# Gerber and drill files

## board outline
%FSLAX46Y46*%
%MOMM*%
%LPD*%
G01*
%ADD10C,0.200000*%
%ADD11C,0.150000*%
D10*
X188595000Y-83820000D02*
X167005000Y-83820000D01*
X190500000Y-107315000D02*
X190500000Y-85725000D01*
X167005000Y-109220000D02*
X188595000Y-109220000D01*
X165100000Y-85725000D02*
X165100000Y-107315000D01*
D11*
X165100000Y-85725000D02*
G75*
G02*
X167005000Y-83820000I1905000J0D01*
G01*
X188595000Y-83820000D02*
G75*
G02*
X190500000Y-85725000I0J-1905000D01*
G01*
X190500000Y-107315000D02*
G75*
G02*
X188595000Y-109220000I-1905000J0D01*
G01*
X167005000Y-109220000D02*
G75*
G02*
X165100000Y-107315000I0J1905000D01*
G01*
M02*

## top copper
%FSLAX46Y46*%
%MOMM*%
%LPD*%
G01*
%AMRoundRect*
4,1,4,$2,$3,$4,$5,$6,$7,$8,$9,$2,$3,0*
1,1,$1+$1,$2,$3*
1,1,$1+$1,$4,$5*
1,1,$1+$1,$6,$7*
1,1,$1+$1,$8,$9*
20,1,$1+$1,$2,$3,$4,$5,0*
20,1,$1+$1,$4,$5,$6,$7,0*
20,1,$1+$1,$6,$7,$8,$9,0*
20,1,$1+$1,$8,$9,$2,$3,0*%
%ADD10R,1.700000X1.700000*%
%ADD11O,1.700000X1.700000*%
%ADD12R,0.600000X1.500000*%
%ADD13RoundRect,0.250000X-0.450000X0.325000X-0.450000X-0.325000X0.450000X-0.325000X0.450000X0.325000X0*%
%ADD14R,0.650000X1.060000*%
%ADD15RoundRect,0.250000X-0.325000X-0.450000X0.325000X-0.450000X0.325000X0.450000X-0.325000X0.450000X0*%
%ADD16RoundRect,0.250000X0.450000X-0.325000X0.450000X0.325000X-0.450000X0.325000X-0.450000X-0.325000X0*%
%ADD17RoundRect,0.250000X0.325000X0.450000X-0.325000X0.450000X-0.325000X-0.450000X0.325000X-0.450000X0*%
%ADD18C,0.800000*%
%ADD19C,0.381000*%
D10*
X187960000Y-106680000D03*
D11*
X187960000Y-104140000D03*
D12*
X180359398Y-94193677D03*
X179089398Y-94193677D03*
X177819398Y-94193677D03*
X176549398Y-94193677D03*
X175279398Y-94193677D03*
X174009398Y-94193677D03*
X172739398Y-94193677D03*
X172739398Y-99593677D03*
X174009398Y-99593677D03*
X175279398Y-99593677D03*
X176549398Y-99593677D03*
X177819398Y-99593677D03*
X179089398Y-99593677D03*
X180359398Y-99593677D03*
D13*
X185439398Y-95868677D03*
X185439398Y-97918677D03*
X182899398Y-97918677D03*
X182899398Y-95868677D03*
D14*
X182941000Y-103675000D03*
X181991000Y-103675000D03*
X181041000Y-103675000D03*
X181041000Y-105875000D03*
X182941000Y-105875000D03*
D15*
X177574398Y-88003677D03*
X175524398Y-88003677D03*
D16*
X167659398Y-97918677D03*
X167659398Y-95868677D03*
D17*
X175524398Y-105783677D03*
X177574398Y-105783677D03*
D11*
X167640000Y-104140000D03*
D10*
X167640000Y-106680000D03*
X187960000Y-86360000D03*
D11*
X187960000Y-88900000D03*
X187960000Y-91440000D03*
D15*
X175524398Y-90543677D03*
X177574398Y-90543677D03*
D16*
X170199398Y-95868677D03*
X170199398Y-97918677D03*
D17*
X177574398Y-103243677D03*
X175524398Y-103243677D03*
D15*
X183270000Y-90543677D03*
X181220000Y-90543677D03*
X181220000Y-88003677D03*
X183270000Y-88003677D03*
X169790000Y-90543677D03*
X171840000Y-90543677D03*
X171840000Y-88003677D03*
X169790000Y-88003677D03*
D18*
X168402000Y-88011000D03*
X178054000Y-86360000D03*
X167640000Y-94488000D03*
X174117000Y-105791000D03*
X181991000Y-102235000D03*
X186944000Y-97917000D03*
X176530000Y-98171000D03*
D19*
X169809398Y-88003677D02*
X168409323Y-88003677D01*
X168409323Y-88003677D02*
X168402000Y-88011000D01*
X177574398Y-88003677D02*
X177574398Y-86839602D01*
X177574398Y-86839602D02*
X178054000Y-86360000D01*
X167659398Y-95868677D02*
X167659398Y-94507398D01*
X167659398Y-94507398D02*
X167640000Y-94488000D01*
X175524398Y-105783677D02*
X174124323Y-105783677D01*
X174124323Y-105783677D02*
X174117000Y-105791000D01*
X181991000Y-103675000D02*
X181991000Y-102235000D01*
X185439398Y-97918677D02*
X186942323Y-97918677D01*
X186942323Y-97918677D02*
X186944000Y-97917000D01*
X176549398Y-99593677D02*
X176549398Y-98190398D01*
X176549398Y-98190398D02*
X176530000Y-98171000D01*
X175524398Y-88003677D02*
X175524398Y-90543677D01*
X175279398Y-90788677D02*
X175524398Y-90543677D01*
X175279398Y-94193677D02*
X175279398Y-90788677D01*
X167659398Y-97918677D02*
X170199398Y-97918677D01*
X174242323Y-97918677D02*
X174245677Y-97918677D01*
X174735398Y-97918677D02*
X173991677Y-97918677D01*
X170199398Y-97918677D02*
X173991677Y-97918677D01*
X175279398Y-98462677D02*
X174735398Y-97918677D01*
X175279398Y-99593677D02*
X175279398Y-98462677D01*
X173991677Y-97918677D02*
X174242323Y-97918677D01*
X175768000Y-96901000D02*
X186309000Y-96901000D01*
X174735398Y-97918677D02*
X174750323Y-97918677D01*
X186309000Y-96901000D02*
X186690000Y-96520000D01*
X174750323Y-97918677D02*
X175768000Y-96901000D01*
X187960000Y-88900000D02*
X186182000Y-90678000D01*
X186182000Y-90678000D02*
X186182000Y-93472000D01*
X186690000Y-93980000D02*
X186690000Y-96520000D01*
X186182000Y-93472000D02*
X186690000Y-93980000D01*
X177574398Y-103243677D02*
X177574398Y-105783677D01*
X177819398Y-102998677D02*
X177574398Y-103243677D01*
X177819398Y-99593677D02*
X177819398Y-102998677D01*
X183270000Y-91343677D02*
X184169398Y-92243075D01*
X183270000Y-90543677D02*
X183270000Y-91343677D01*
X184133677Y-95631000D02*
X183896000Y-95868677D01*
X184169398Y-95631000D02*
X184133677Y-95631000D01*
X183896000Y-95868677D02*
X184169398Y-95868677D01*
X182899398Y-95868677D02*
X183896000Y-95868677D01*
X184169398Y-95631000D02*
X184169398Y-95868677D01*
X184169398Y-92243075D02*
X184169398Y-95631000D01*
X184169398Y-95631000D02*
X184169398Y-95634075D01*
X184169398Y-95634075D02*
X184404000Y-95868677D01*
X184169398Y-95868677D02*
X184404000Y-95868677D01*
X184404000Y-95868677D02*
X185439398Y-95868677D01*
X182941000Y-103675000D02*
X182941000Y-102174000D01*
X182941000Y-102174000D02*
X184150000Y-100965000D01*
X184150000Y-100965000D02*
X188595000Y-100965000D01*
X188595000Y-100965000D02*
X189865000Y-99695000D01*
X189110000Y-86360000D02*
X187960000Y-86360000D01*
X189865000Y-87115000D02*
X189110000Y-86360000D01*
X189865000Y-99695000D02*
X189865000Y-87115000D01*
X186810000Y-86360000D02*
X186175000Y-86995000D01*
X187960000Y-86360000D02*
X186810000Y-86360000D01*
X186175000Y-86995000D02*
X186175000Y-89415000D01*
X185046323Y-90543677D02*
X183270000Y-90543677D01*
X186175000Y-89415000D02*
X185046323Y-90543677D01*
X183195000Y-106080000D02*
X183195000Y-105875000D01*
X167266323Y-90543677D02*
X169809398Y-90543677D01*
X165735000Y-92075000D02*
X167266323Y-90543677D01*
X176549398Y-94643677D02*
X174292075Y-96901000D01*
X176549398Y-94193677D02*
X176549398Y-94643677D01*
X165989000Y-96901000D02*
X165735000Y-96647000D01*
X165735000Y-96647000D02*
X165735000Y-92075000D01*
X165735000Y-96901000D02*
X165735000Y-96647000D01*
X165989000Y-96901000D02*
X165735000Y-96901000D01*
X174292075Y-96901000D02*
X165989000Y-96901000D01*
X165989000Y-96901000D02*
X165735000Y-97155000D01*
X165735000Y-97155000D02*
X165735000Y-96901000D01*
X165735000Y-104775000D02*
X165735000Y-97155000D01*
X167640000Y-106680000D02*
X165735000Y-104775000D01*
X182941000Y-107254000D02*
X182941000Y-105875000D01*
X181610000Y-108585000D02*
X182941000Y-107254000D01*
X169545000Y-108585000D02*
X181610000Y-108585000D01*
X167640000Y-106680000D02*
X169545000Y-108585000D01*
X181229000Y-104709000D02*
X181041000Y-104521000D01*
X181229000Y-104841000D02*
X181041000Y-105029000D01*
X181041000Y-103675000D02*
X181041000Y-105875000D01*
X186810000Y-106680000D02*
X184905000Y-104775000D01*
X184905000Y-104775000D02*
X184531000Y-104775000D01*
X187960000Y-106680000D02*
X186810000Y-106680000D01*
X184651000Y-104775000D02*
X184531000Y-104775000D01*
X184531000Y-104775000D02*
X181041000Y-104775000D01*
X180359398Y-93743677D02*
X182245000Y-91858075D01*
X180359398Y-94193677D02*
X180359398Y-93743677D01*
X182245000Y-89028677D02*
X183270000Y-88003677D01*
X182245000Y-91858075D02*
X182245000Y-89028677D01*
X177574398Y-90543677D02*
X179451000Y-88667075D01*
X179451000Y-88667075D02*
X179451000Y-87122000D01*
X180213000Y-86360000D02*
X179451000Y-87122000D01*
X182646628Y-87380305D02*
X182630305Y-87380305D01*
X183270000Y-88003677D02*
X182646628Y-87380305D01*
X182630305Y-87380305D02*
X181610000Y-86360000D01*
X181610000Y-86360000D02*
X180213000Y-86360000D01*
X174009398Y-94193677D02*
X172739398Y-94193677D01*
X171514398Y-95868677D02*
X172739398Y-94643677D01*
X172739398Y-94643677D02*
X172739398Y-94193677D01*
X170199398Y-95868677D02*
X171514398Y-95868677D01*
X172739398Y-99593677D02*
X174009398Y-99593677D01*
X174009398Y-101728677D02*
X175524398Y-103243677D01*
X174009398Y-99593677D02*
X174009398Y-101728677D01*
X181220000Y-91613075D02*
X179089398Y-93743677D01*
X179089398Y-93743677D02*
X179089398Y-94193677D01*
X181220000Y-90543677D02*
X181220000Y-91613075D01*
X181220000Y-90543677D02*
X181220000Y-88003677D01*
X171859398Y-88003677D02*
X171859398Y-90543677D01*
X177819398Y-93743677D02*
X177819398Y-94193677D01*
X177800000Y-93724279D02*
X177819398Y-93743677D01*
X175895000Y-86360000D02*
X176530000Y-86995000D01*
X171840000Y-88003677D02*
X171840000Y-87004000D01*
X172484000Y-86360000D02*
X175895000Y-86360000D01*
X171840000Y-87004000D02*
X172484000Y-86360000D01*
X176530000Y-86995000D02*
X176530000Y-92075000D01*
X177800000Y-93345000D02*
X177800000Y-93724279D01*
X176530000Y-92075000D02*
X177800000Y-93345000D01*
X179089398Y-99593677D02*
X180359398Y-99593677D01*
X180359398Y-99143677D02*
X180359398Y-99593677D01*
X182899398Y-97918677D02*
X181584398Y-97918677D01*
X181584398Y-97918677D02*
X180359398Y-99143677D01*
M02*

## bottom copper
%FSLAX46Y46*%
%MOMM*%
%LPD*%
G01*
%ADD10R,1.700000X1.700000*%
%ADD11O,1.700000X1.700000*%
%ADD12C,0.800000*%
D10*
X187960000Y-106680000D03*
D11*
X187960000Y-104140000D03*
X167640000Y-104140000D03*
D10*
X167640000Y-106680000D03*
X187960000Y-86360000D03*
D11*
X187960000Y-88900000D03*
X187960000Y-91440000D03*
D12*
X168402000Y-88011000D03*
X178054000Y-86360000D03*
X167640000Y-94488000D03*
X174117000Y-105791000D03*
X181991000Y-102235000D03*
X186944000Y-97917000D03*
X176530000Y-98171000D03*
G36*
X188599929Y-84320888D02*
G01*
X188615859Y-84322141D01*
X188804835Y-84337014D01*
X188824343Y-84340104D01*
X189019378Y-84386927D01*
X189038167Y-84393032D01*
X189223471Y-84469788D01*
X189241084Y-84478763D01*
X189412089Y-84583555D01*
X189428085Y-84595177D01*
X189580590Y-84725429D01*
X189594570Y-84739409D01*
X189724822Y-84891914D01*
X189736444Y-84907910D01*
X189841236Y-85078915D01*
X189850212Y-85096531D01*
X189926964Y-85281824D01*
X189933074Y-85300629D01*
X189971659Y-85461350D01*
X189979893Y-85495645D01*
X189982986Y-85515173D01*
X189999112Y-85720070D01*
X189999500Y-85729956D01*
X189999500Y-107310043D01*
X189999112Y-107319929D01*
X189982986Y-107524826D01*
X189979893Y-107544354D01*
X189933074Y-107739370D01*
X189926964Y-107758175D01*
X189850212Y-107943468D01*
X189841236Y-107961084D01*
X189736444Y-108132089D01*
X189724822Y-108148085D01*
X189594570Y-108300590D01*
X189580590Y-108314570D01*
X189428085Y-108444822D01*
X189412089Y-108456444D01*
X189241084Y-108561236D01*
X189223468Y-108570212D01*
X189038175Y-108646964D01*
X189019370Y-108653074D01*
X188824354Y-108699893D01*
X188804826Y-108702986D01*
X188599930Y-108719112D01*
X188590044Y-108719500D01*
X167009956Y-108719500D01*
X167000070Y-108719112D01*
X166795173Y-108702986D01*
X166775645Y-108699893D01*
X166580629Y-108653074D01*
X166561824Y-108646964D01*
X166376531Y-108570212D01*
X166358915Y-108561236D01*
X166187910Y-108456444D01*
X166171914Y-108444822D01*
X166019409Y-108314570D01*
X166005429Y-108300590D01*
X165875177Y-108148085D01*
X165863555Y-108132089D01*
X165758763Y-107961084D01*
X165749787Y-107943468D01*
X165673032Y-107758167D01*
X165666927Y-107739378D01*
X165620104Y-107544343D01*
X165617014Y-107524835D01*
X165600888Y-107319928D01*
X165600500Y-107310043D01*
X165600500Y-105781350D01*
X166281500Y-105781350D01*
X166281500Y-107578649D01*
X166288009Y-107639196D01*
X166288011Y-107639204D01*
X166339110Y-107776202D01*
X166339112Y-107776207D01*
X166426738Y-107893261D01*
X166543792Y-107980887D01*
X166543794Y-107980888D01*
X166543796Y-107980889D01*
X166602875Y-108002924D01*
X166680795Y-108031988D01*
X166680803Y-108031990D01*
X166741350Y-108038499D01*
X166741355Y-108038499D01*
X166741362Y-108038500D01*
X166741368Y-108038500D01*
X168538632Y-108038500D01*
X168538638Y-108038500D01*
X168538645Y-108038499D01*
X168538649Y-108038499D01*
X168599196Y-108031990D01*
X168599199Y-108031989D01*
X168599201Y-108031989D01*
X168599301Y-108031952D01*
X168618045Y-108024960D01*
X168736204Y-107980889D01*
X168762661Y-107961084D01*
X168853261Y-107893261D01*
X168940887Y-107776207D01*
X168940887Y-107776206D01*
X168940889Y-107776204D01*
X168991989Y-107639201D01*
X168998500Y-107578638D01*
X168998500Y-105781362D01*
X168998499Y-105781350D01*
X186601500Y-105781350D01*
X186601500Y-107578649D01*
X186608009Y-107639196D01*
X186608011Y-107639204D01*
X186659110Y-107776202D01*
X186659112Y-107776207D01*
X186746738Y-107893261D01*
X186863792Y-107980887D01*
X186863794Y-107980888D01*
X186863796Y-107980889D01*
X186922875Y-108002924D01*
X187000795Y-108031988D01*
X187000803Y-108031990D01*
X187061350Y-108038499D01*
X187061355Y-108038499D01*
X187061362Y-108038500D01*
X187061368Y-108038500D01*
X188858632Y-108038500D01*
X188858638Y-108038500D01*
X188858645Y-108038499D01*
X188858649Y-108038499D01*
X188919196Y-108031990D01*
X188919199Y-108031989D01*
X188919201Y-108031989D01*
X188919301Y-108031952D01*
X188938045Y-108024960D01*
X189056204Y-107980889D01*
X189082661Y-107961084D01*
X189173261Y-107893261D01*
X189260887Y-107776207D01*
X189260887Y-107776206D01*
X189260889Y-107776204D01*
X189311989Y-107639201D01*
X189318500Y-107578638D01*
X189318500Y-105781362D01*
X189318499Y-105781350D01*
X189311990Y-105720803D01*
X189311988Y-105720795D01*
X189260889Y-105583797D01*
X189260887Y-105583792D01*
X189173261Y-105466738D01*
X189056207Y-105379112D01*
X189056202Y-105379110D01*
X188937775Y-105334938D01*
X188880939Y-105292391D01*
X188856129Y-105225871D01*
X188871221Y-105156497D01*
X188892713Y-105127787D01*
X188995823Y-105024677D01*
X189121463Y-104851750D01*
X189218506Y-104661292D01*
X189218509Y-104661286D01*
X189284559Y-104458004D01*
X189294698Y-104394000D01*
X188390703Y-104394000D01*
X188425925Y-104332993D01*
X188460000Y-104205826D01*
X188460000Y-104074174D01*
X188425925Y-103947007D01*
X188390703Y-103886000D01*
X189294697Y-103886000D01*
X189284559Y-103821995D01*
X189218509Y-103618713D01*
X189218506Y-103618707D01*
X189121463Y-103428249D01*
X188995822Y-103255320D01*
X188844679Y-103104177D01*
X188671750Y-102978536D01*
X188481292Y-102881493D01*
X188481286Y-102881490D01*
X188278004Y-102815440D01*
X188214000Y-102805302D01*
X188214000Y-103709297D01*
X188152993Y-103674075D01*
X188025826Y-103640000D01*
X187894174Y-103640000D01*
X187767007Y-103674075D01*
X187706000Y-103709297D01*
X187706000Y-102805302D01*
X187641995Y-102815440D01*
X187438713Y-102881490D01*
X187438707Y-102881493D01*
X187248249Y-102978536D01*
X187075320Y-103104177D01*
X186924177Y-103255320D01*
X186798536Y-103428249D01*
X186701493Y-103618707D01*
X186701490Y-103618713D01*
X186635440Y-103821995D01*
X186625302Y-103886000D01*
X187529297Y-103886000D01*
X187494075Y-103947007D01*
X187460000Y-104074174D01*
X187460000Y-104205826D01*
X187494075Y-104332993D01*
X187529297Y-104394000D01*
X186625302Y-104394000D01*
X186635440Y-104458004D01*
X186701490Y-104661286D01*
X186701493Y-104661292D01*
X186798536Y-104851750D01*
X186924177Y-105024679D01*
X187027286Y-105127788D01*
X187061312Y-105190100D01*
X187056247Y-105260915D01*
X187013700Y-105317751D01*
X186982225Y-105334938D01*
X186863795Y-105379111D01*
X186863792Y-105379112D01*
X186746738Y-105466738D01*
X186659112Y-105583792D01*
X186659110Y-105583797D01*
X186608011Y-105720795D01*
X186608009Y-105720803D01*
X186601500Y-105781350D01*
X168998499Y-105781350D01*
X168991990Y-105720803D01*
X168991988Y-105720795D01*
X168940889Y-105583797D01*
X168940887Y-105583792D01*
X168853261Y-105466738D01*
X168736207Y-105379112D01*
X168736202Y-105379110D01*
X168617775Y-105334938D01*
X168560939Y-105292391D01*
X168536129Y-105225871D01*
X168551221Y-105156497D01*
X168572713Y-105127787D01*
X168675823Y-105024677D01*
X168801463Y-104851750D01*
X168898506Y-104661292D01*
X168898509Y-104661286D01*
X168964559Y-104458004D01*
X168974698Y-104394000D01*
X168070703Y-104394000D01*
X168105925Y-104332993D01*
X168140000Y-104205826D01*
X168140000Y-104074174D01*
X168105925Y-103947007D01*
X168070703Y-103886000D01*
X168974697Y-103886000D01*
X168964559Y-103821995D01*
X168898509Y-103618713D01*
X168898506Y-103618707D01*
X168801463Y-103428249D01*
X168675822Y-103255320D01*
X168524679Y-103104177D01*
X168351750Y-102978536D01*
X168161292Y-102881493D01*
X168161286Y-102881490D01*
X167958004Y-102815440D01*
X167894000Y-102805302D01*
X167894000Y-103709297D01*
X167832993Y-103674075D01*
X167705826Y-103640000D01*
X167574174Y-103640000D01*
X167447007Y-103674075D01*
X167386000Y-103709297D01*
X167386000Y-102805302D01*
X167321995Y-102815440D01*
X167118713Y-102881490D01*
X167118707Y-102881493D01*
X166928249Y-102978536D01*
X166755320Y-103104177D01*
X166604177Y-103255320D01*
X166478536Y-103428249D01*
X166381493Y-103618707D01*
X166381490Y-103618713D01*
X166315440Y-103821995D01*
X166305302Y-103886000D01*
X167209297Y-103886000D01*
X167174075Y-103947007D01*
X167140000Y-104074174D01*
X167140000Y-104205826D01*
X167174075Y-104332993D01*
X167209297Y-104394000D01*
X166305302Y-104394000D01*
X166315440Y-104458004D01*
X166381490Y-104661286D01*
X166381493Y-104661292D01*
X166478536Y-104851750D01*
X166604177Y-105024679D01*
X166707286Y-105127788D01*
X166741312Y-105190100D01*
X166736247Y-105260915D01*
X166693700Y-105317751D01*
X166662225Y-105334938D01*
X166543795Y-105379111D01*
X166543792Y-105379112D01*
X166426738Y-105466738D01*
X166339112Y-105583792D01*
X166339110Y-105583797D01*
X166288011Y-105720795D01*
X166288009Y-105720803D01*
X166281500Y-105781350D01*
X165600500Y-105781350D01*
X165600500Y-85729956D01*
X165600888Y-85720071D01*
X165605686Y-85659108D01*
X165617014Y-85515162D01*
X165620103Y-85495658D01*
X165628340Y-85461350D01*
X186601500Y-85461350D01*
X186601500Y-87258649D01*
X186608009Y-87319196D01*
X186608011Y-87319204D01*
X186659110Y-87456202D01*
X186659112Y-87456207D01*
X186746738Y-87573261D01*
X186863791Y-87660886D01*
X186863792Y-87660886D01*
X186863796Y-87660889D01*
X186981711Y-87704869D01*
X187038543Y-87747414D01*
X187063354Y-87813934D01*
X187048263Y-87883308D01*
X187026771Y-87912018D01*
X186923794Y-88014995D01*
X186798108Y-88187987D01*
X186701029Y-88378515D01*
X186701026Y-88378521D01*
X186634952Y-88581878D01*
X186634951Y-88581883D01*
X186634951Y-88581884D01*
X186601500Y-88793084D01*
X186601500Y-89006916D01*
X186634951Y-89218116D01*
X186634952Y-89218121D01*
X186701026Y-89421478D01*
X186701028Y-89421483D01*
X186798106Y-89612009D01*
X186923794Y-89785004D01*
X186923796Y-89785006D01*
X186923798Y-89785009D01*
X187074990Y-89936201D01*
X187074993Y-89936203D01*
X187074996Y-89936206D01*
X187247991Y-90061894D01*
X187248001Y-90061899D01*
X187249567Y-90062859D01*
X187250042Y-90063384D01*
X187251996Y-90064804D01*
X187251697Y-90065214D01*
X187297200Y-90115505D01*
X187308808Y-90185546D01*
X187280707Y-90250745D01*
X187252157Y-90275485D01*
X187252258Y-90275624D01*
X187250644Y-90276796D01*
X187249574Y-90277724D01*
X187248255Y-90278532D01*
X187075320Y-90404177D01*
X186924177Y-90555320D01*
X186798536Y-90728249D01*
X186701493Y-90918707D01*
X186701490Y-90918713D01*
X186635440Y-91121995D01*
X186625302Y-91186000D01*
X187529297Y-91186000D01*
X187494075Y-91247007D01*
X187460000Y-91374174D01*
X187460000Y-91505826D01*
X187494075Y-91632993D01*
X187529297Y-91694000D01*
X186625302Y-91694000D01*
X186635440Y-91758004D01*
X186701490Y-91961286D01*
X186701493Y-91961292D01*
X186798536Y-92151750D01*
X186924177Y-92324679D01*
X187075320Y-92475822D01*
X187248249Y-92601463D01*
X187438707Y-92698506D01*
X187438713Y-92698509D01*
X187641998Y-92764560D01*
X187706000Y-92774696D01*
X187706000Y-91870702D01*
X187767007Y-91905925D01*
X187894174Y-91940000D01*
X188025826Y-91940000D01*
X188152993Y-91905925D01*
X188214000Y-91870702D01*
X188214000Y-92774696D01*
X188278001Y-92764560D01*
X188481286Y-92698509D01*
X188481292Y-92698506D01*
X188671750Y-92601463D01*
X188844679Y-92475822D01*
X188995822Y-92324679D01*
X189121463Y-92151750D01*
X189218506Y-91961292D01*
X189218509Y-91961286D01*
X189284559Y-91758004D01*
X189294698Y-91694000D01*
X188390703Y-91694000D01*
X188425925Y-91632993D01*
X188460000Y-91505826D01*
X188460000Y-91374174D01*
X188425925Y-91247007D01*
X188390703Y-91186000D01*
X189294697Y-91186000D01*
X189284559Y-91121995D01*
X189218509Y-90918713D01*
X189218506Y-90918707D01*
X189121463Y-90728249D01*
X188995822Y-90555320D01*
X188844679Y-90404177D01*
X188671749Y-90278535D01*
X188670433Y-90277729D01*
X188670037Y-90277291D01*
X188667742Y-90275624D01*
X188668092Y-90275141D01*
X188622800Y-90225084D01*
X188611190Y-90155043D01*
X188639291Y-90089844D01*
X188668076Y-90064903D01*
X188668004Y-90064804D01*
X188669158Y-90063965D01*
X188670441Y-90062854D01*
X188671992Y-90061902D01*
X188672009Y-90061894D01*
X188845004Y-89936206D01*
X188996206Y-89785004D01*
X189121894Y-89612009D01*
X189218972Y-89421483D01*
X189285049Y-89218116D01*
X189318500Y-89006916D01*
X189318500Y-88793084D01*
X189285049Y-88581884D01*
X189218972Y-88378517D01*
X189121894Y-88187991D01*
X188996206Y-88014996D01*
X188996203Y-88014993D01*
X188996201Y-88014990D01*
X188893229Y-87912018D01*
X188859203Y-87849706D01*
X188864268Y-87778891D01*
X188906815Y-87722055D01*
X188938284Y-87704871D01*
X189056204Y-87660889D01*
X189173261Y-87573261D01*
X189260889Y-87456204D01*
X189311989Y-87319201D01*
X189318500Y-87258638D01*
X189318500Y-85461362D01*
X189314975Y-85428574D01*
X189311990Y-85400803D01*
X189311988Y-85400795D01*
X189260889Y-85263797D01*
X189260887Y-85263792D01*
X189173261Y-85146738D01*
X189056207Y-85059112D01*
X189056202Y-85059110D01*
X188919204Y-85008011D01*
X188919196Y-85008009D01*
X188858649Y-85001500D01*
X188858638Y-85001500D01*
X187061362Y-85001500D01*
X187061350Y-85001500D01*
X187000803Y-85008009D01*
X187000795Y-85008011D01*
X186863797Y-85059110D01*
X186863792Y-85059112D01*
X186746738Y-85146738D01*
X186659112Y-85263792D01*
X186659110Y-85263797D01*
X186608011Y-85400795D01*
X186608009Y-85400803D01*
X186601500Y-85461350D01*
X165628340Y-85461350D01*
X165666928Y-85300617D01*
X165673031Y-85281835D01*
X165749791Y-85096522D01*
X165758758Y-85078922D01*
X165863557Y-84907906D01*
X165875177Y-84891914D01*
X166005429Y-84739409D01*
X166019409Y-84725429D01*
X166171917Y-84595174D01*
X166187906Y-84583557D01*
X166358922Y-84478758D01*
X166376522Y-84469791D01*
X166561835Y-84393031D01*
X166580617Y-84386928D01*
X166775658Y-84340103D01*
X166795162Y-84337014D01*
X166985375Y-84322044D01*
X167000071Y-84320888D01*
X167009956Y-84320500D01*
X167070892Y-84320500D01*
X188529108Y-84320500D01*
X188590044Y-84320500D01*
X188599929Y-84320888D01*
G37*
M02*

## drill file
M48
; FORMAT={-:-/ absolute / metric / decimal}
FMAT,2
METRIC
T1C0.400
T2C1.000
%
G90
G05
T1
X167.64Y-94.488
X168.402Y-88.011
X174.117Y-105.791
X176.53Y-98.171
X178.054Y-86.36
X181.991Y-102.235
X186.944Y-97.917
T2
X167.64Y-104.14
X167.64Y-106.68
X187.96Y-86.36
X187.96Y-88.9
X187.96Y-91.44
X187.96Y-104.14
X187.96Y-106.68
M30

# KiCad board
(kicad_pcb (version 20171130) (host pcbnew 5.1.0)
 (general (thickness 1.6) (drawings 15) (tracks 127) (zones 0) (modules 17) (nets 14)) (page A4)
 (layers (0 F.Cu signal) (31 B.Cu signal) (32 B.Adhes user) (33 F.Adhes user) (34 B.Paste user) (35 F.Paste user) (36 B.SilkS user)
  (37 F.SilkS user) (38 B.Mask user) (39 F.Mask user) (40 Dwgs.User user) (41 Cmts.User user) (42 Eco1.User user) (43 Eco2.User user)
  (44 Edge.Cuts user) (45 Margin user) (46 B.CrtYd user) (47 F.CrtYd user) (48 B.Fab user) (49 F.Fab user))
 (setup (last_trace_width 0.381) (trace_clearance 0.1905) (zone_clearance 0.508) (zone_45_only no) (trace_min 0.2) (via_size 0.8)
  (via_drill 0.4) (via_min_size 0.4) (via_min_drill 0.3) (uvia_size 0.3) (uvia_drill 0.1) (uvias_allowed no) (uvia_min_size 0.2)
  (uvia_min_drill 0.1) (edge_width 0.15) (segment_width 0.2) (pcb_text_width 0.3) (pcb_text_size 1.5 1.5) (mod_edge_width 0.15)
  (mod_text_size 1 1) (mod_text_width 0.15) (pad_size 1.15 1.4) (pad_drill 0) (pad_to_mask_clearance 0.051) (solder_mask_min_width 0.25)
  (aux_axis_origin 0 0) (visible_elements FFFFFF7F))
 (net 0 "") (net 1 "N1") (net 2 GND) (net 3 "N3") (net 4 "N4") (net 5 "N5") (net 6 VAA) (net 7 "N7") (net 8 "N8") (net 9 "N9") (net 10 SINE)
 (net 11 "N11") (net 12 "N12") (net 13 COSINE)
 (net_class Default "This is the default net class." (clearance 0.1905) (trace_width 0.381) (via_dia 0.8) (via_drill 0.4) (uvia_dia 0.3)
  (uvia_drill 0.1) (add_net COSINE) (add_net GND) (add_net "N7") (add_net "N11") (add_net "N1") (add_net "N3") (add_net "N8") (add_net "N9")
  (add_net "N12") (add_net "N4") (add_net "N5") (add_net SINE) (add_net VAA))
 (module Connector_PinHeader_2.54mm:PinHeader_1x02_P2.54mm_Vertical (layer F.Cu) (at 187.96 106.68 180)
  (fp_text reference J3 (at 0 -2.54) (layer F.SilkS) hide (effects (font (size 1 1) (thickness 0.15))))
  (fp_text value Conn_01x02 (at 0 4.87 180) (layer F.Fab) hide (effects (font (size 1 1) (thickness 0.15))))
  (pad 1 thru_hole rect (at 0 0 180) (size 1.7 1.7) (drill 1) (layers *.Cu *.Mask) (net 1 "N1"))
  (pad 2 thru_hole oval (at 0 2.54 180) (size 1.7 1.7) (drill 1) (layers *.Cu *.Mask) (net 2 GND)))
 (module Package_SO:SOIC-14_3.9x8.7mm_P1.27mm (layer F.Cu) (at 176.549398 96.893677 270)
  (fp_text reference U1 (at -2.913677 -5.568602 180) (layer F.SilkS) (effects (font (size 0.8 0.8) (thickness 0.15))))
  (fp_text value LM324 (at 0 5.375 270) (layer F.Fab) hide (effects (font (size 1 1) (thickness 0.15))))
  (pad 1 smd rect (at -2.7 -3.81 270) (size 1.5 0.6) (layers F.Cu F.Paste F.Mask) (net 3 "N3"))
  (pad 2 smd rect (at -2.7 -2.54 270) (size 1.5 0.6) (layers F.Cu F.Paste F.Mask) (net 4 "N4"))
  (pad 3 smd rect (at -2.7 -1.27 270) (size 1.5 0.6) (layers F.Cu F.Paste F.Mask) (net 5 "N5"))
  (pad 4 smd rect (at -2.7 0 270) (size 1.5 0.6) (layers F.Cu F.Paste F.Mask) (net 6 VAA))
  (pad 5 smd rect (at -2.7 1.27 270) (size 1.5 0.6) (layers F.Cu F.Paste F.Mask) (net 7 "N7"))
  (pad 6 smd rect (at -2.7 2.54 270) (size 1.5 0.6) (layers F.Cu F.Paste F.Mask) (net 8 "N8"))
  (pad 7 smd rect (at -2.7 3.81 270) (size 1.5 0.6) (layers F.Cu F.Paste F.Mask) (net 8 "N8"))
  (pad 8 smd rect (at 2.7 3.81 270) (size 1.5 0.6) (layers F.Cu F.Paste F.Mask) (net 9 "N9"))
  (pad 9 smd rect (at 2.7 2.54 270) (size 1.5 0.6) (layers F.Cu F.Paste F.Mask) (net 9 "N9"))
  (pad 10 smd rect (at 2.7 1.27 270) (size 1.5 0.6) (layers F.Cu F.Paste F.Mask) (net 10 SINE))
  (pad 11 smd rect (at 2.7 0 270) (size 1.5 0.6) (layers F.Cu F.Paste F.Mask) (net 2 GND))
  (pad 12 smd rect (at 2.7 -1.27 270) (size 1.5 0.6) (layers F.Cu F.Paste F.Mask) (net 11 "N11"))
  (pad 13 smd rect (at 2.7 -2.54 270) (size 1.5 0.6) (layers F.Cu F.Paste F.Mask) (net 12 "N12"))
  (pad 14 smd rect (at 2.7 -3.81 270) (size 1.5 0.6) (layers F.Cu F.Paste F.Mask) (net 12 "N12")))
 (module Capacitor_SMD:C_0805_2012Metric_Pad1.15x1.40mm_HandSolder (layer F.Cu) (at 185.439398 96.893677 270)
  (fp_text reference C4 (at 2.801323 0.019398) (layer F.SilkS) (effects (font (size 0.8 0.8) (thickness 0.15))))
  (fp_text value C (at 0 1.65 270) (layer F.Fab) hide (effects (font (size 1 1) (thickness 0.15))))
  (pad 1 smd roundrect (at -1.025 0 270) (size 1.15 1.4) (layers F.Cu F.Paste F.Mask) (roundrect_rratio 0.217391) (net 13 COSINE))
  (pad 2 smd roundrect (at 1.025 0 270) (size 1.15 1.4) (layers F.Cu F.Paste F.Mask) (roundrect_rratio 0.217391) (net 2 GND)))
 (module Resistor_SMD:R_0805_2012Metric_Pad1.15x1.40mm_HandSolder (layer F.Cu) (at 182.899398 96.893677 270)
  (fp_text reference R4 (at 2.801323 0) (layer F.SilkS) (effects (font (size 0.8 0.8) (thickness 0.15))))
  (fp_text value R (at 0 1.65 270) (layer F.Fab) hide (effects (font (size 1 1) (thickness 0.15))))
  (pad 2 smd roundrect (at 1.025 0 270) (size 1.15 1.4) (layers F.Cu F.Paste F.Mask) (roundrect_rratio 0.217391) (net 12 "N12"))
  (pad 1 smd roundrect (at -1.025 0 270) (size 1.15 1.4) (layers F.Cu F.Paste F.Mask) (roundrect_rratio 0.217391) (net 13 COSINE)))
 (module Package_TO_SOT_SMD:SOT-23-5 (layer F.Cu) (at 181.991 104.775 270)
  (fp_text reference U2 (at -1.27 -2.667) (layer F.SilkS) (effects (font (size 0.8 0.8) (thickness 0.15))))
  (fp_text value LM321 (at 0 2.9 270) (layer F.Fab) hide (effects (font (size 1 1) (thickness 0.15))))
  (pad 1 smd rect (at -1.1 -0.95 270) (size 1.06 0.65) (layers F.Cu F.Paste F.Mask) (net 13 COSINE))
  (pad 2 smd rect (at -1.1 0 270) (size 1.06 0.65) (layers F.Cu F.Paste F.Mask) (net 2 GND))
  (pad 3 smd rect (at -1.1 0.95 270) (size 1.06 0.65) (layers F.Cu F.Paste F.Mask) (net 1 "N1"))
  (pad 4 smd rect (at 1.1 0.95 270) (size 1.06 0.65) (layers F.Cu F.Paste F.Mask) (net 1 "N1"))
  (pad 5 smd rect (at 1.1 -0.95 270) (size 1.06 0.65) (layers F.Cu F.Paste F.Mask) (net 6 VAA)))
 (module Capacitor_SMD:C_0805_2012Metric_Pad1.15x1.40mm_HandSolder (layer F.Cu) (at 176.549398 88.003677)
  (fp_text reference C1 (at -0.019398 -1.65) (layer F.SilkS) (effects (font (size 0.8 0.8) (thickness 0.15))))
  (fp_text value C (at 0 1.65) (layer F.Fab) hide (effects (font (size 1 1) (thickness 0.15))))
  (pad 2 smd roundrect (at 1.025 0) (size 1.15 1.4) (layers F.Cu F.Paste F.Mask) (roundrect_rratio 0.217391) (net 2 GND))
  (pad 1 smd roundrect (at -1.025 0) (size 1.15 1.4) (layers F.Cu F.Paste F.Mask) (roundrect_rratio 0.217391) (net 7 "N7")))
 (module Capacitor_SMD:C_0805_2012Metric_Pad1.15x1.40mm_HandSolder (layer F.Cu) (at 167.659398 96.893677 90)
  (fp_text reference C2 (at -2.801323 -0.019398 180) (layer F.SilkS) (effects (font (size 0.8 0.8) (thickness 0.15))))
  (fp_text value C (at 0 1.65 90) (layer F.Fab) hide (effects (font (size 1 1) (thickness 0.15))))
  (pad 1 smd roundrect (at -1.025 0 90) (size 1.15 1.4) (layers F.Cu F.Paste F.Mask) (roundrect_rratio 0.217391) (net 10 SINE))
  (pad 2 smd roundrect (at 1.025 0 90) (size 1.15 1.4) (layers F.Cu F.Paste F.Mask) (roundrect_rratio 0.217391) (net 2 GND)))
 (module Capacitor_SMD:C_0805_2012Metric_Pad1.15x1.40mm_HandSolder (layer F.Cu) (at 176.549398 105.783677 180)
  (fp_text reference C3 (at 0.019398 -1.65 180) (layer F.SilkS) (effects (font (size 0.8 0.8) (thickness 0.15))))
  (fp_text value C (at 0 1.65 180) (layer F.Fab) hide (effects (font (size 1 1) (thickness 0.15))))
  (pad 2 smd roundrect (at 1.025 0 180) (size 1.15 1.4) (layers F.Cu F.Paste F.Mask) (roundrect_rratio 0.217391) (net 2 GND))
  (pad 1 smd roundrect (at -1.025 0 180) (size 1.15 1.4) (layers F.Cu F.Paste F.Mask) (roundrect_rratio 0.217391) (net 11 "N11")))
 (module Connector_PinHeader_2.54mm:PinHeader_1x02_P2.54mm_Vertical (layer F.Cu) (at 167.64 106.68 180)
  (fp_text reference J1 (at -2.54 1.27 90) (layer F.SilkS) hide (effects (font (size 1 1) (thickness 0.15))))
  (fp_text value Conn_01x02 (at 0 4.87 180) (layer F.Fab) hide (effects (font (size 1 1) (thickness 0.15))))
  (pad 2 thru_hole oval (at 0 2.54 180) (size 1.7 1.7) (drill 1) (layers *.Cu *.Mask) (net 2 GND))
  (pad 1 thru_hole rect (at 0 0 180) (size 1.7 1.7) (drill 1) (layers *.Cu *.Mask) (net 6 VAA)))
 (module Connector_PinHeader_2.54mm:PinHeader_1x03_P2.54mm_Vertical (layer F.Cu) (at 187.96 86.36)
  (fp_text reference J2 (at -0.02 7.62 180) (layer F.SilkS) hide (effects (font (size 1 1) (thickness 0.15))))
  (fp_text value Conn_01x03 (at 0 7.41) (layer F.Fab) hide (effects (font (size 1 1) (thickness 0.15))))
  (pad 1 thru_hole rect (at 0 0) (size 1.7 1.7) (drill 1) (layers *.Cu *.Mask) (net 13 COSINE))
  (pad 2 thru_hole oval (at 0 2.54) (size 1.7 1.7) (drill 1) (layers *.Cu *.Mask) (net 10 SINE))
  (pad 3 thru_hole oval (at 0 5.08) (size 1.7 1.7) (drill 1) (layers *.Cu *.Mask) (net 2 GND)))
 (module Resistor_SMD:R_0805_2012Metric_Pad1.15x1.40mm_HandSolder (layer F.Cu) (at 176.549398 90.543677)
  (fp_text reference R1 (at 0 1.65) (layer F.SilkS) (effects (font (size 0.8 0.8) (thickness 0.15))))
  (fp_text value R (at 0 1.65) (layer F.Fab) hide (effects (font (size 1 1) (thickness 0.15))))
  (pad 1 smd roundrect (at -1.025 0) (size 1.15 1.4) (layers F.Cu F.Paste F.Mask) (roundrect_rratio 0.217391) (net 7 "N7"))
  (pad 2 smd roundrect (at 1.025 0) (size 1.15 1.4) (layers F.Cu F.Paste F.Mask) (roundrect_rratio 0.217391) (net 3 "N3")))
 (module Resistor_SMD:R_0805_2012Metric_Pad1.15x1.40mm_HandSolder (layer F.Cu) (at 170.199398 96.893677 90)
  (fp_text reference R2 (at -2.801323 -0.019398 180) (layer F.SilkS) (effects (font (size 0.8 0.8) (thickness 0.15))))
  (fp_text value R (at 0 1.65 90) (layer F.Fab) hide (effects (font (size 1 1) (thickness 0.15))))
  (pad 2 smd roundrect (at 1.025 0 90) (size 1.15 1.4) (layers F.Cu F.Paste F.Mask) (roundrect_rratio 0.217391) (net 8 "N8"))
  (pad 1 smd roundrect (at -1.025 0 90) (size 1.15 1.4) (layers F.Cu F.Paste F.Mask) (roundrect_rratio 0.217391) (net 10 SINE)))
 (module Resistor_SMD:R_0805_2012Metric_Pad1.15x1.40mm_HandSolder (layer F.Cu) (at 176.549398 103.243677 180)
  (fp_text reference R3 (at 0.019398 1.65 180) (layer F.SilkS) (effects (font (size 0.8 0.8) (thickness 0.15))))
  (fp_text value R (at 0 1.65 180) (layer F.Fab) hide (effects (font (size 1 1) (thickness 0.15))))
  (pad 1 smd roundrect (at -1.025 0 180) (size 1.15 1.4) (layers F.Cu F.Paste F.Mask) (roundrect_rratio 0.217391) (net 11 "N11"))
  (pad 2 smd roundrect (at 1.025 0 180) (size 1.15 1.4) (layers F.Cu F.Paste F.Mask) (roundrect_rratio 0.217391) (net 9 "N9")))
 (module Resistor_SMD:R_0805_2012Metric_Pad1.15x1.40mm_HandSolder (layer F.Cu) (at 182.245 90.543677)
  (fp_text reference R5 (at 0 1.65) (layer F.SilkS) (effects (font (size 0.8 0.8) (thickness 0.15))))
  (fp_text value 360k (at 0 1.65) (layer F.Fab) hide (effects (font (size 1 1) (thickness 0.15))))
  (pad 2 smd roundrect (at 1.025 0) (size 1.15 1.4) (layers F.Cu F.Paste F.Mask) (roundrect_rratio 0.217391) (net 13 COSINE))
  (pad 1 smd roundrect (at -1.025 0) (size 1.15 1.4) (layers F.Cu F.Paste F.Mask) (roundrect_rratio 0.217391) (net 4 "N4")))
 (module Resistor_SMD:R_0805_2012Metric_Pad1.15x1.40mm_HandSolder (layer F.Cu) (at 182.245 88.003677)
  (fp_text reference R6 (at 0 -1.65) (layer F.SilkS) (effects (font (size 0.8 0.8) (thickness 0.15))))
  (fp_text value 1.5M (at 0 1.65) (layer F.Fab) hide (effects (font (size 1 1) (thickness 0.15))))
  (pad 1 smd roundrect (at -1.025 0) (size 1.15 1.4) (layers F.Cu F.Paste F.Mask) (roundrect_rratio 0.217391) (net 4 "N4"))
  (pad 2 smd roundrect (at 1.025 0) (size 1.15 1.4) (layers F.Cu F.Paste F.Mask) (roundrect_rratio 0.217391) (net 3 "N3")))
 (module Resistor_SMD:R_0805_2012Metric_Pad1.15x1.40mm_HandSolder (layer F.Cu) (at 170.815 90.543677)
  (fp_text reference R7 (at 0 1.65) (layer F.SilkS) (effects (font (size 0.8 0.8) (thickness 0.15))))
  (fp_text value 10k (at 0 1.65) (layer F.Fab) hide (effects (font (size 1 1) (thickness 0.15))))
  (pad 1 smd roundrect (at -1.025 0) (size 1.15 1.4) (layers F.Cu F.Paste F.Mask) (roundrect_rratio 0.217391) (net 6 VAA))
  (pad 2 smd roundrect (at 1.025 0) (size 1.15 1.4) (layers F.Cu F.Paste F.Mask) (roundrect_rratio 0.217391) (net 5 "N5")))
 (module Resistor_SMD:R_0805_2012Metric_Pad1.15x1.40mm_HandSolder (layer F.Cu) (at 170.815 88.003677)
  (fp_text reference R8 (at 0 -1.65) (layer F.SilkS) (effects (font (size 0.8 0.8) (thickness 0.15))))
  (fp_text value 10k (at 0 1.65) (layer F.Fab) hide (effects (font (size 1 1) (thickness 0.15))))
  (pad 2 smd roundrect (at 1.025 0) (size 1.15 1.4) (layers F.Cu F.Paste F.Mask) (roundrect_rratio 0.217391) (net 5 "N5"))
  (pad 1 smd roundrect (at -1.025 0) (size 1.15 1.4) (layers F.Cu F.Paste F.Mask) (roundrect_rratio 0.217391) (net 2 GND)))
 (gr_line (start 188.595 83.82) (end 167.005 83.82) (layer Edge.Cuts) (width 0.2))
 (gr_line (start 190.5 107.315) (end 190.5 85.725) (layer Edge.Cuts) (width 0.2))
 (gr_line (start 167.005 109.22) (end 188.595 109.22) (layer Edge.Cuts) (width 0.2))
 (gr_line (start 165.1 85.725) (end 165.1 107.315) (layer Edge.Cuts) (width 0.2))
 (gr_arc (start 167.005 85.725) (end 167.005 83.82) (angle -90) (layer Edge.Cuts) (width 0.15))
 (gr_arc (start 188.595 85.725) (end 190.5 85.725) (angle -90) (layer Edge.Cuts) (width 0.15))
 (gr_arc (start 188.595 107.315) (end 188.595 109.22) (angle -90) (layer Edge.Cuts) (width 0.15))
 (gr_arc (start 167.005 107.315) (end 165.1 107.315) (angle -90) (layer Edge.Cuts) (width 0.15))
 (via (at 168.402 88.011) (size 0.8) (drill 0.4) (layers F.Cu B.Cu) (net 2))
 (segment (start 169.809398 88.003677) (end 168.409323 88.003677) (width 0.381) (layer F.Cu) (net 2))
 (segment (start 168.409323 88.003677) (end 168.402 88.011) (width 0.381) (layer F.Cu) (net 2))
 (via (at 178.054 86.36) (size 0.8) (drill 0.4) (layers F.Cu B.Cu) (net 2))
 (segment (start 177.574398 88.003677) (end 177.574398 86.839602) (width 0.381) (layer F.Cu) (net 2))
 (segment (start 177.574398 86.839602) (end 178.054 86.36) (width 0.381) (layer F.Cu) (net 2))
 (segment (start 167.659398 95.868677) (end 167.659398 94.507398) (width 0.381) (layer F.Cu) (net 2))
 (via (at 167.64 94.488) (size 0.8) (drill 0.4) (layers F.Cu B.Cu) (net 2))
 (segment (start 167.659398 94.507398) (end 167.64 94.488) (width 0.381) (layer F.Cu) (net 2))
 (via (at 174.117 105.791) (size 0.8) (drill 0.4) (layers F.Cu B.Cu) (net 2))
 (segment (start 175.524398 105.783677) (end 174.124323 105.783677) (width 0.381) (layer F.Cu) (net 2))
 (segment (start 174.124323 105.783677) (end 174.117 105.791) (width 0.381) (layer F.Cu) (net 2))
 (via (at 181.991 102.235) (size 0.8) (drill 0.4) (layers F.Cu B.Cu) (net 2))
 (segment (start 181.991 103.675) (end 181.991 102.235) (width 0.381) (layer F.Cu) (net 2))
 (via (at 186.944 97.917) (size 0.8) (drill 0.4) (layers F.Cu B.Cu) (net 2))
 (segment (start 185.439398 97.918677) (end 186.942323 97.918677) (width 0.381) (layer F.Cu) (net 2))
 (segment (start 186.942323 97.918677) (end 186.944 97.917) (width 0.381) (layer F.Cu) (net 2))
 (via (at 176.53 98.171) (size 0.8) (drill 0.4) (layers F.Cu B.Cu) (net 2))
 (segment (start 176.549398 99.593677) (end 176.549398 98.190398) (width 0.381) (layer F.Cu) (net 2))
 (segment (start 176.549398 98.190398) (end 176.53 98.171) (width 0.381) (layer F.Cu) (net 2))
 (segment (start 175.524398 88.003677) (end 175.524398 90.543677) (width 0.381) (layer F.Cu) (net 7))
 (segment (start 175.279398 90.788677) (end 175.524398 90.543677) (width 0.381) (layer F.Cu) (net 7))
 (segment (start 175.279398 94.193677) (end 175.279398 90.788677) (width 0.381) (layer F.Cu) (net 7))
 (segment (start 167.659398 97.918677) (end 170.199398 97.918677) (width 0.381) (layer F.Cu) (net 10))
 (segment (start 174.242323 97.918677) (end 174.245677 97.918677) (width 0.381) (layer F.Cu) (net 10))
 (segment (start 174.735398 97.918677) (end 173.991677 97.918677) (width 0.381) (layer F.Cu) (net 10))
 (segment (start 170.199398 97.918677) (end 173.991677 97.918677) (width 0.381) (layer F.Cu) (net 10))
 (segment (start 175.279398 98.462677) (end 174.735398 97.918677) (width 0.381) (layer F.Cu) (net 10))
 (segment (start 175.279398 99.593677) (end 175.279398 98.462677) (width 0.381) (layer F.Cu) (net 10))
 (segment (start 173.991677 97.918677) (end 174.242323 97.918677) (width 0.381) (layer F.Cu) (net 10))
 (segment (start 175.768 96.901) (end 186.309 96.901) (width 0.381) (layer F.Cu) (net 10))
 (segment (start 174.735398 97.918677) (end 174.750323 97.918677) (width 0.381) (layer F.Cu) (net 10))
 (segment (start 186.309 96.901) (end 186.69 96.52) (width 0.381) (layer F.Cu) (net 10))
 (segment (start 174.750323 97.918677) (end 175.768 96.901) (width 0.381) (layer F.Cu) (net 10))
 (segment (start 187.96 88.9) (end 186.182 90.678) (width 0.381) (layer F.Cu) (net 10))
 (segment (start 186.182 90.678) (end 186.182 93.472) (width 0.381) (layer F.Cu) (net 10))
 (segment (start 186.69 93.98) (end 186.69 96.52) (width 0.381) (layer F.Cu) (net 10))
 (segment (start 186.182 93.472) (end 186.69 93.98) (width 0.381) (layer F.Cu) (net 10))
 (segment (start 177.574398 103.243677) (end 177.574398 105.783677) (width 0.381) (layer F.Cu) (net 11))
 (segment (start 177.819398 102.998677) (end 177.574398 103.243677) (width 0.381) (layer F.Cu) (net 11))
 (segment (start 177.819398 99.593677) (end 177.819398 102.998677) (width 0.381) (layer F.Cu) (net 11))
 (segment (start 183.27 91.343677) (end 184.169398 92.243075) (width 0.381) (layer F.Cu) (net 13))
 (segment (start 183.27 90.543677) (end 183.27 91.343677) (width 0.381) (layer F.Cu) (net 13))
 (segment (start 184.133677 95.631) (end 183.896 95.868677) (width 0.381) (layer F.Cu) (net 13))
 (segment (start 184.169398 95.631) (end 184.133677 95.631) (width 0.381) (layer F.Cu) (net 13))
 (segment (start 183.896 95.868677) (end 184.169398 95.868677) (width 0.381) (layer F.Cu) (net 13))
 (segment (start 182.899398 95.868677) (end 183.896 95.868677) (width 0.381) (layer F.Cu) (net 13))
 (segment (start 184.169398 95.631) (end 184.169398 95.868677) (width 0.381) (layer F.Cu) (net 13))
 (segment (start 184.169398 92.243075) (end 184.169398 95.631) (width 0.381) (layer F.Cu) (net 13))
 (segment (start 184.169398 95.631) (end 184.169398 95.634075) (width 0.381) (layer F.Cu) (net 13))
 (segment (start 184.169398 95.634075) (end 184.404 95.868677) (width 0.381) (layer F.Cu) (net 13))
 (segment (start 184.169398 95.868677) (end 184.404 95.868677) (width 0.381) (layer F.Cu) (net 13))
 (segment (start 184.404 95.868677) (end 185.439398 95.868677) (width 0.381) (layer F.Cu) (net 13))
 (segment (start 182.941 103.675) (end 182.941 102.174) (width 0.381) (layer F.Cu) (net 13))
 (segment (start 182.941 102.174) (end 184.15 100.965) (width 0.381) (layer F.Cu) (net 13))
 (segment (start 184.15 100.965) (end 188.595 100.965) (width 0.381) (layer F.Cu) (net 13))
 (segment (start 188.595 100.965) (end 189.865 99.695) (width 0.381) (layer F.Cu) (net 13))
 (segment (start 189.11 86.36) (end 187.96 86.36) (width 0.381) (layer F.Cu) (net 13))
 (segment (start 189.865 87.115) (end 189.11 86.36) (width 0.381) (layer F.Cu) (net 13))
 (segment (start 189.865 99.695) (end 189.865 87.115) (width 0.381) (layer F.Cu) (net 13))
 (segment (start 186.81 86.36) (end 186.175 86.995) (width 0.381) (layer F.Cu) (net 13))
 (segment (start 187.96 86.36) (end 186.81 86.36) (width 0.381) (layer F.Cu) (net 13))
 (segment (start 186.175 86.995) (end 186.175 89.415) (width 0.381) (layer F.Cu) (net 13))
 (segment (start 185.046323 90.543677) (end 183.27 90.543677) (width 0.381) (layer F.Cu) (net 13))
 (segment (start 186.175 89.415) (end 185.046323 90.543677) (width 0.381) (layer F.Cu) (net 13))
 (segment (start 183.195 106.08) (end 183.195 105.875) (width 0.381) (layer F.Cu) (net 6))
 (segment (start 167.266323 90.543677) (end 169.809398 90.543677) (width 0.381) (layer F.Cu) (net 6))
 (segment (start 165.735 92.075) (end 167.266323 90.543677) (width 0.381) (layer F.Cu) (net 6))
 (segment (start 176.549398 94.643677) (end 174.292075 96.901) (width 0.381) (layer F.Cu) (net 6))
 (segment (start 176.549398 94.193677) (end 176.549398 94.643677) (width 0.381) (layer F.Cu) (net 6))
 (segment (start 165.989 96.901) (end 165.735 96.647) (width 0.381) (layer F.Cu) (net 6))
 (segment (start 165.735 96.647) (end 165.735 92.075) (width 0.381) (layer F.Cu) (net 6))
 (segment (start 165.735 96.901) (end 165.735 96.647) (width 0.381) (layer F.Cu) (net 6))
 (segment (start 165.989 96.901) (end 165.735 96.901) (width 0.381) (layer F.Cu) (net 6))
 (segment (start 174.292075 96.901) (end 165.989 96.901) (width 0.381) (layer F.Cu) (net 6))
 (segment (start 165.989 96.901) (end 165.735 97.155) (width 0.381) (layer F.Cu) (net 6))
 (segment (start 165.735 97.155) (end 165.735 96.901) (width 0.381) (layer F.Cu) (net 6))
 (segment (start 165.735 104.775) (end 165.735 97.155) (width 0.381) (layer F.Cu) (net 6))
 (segment (start 167.64 106.68) (end 165.735 104.775) (width 0.381) (layer F.Cu) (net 6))
 (segment (start 182.941 107.254) (end 182.941 105.875) (width 0.381) (layer F.Cu) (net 6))
 (segment (start 181.61 108.585) (end 182.941 107.254) (width 0.381) (layer F.Cu) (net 6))
 (segment (start 169.545 108.585) (end 181.61 108.585) (width 0.381) (layer F.Cu) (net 6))
 (segment (start 167.64 106.68) (end 169.545 108.585) (width 0.381) (layer F.Cu) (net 6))
 (segment (start 181.229 104.709) (end 181.041 104.521) (width 0.381) (layer F.Cu) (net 1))
 (segment (start 181.229 104.841) (end 181.041 105.029) (width 0.381) (layer F.Cu) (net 1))
 (segment (start 181.041 103.675) (end 181.041 105.875) (width 0.381) (layer F.Cu) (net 1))
 (segment (start 186.81 106.68) (end 184.905 104.775) (width 0.381) (layer F.Cu) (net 1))
 (segment (start 184.905 104.775) (end 184.531 104.775) (width 0.381) (layer F.Cu) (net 1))
 (segment (start 187.96 106.68) (end 186.81 106.68) (width 0.381) (layer F.Cu) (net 1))
 (segment (start 184.651 104.775) (end 184.531 104.775) (width 0.381) (layer F.Cu) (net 1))
 (segment (start 184.531 104.775) (end 181.041 104.775) (width 0.381) (layer F.Cu) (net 1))
 (segment (start 180.359398 93.743677) (end 182.245 91.858075) (width 0.381) (layer F.Cu) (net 3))
 (segment (start 180.359398 94.193677) (end 180.359398 93.743677) (width 0.381) (layer F.Cu) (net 3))
 (segment (start 182.245 89.028677) (end 183.27 88.003677) (width 0.381) (layer F.Cu) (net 3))
 (segment (start 182.245 91.858075) (end 182.245 89.028677) (width 0.381) (layer F.Cu) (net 3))
 (segment (start 177.574398 90.543677) (end 179.451 88.667075) (width 0.381) (layer F.Cu) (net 3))
 (segment (start 179.451 88.667075) (end 179.451 87.122) (width 0.381) (layer F.Cu) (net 3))
 (segment (start 180.213 86.36) (end 179.451 87.122) (width 0.381) (layer F.Cu) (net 3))
 (segment (start 182.646628 87.380305) (end 182.630305 87.380305) (width 0.381) (layer F.Cu) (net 3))
 (segment (start 183.27 88.003677) (end 182.646628 87.380305) (width 0.381) (layer F.Cu) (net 3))
 (segment (start 182.630305 87.380305) (end 181.61 86.36) (width 0.381) (layer F.Cu) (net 3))
 (segment (start 181.61 86.36) (end 180.213 86.36) (width 0.381) (layer F.Cu) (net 3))
 (segment (start 174.009398 94.193677) (end 172.739398 94.193677) (width 0.381) (layer F.Cu) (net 8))
 (segment (start 171.514398 95.868677) (end 172.739398 94.643677) (width 0.381) (layer F.Cu) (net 8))
 (segment (start 172.739398 94.643677) (end 172.739398 94.193677) (width 0.381) (layer F.Cu) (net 8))
 (segment (start 170.199398 95.868677) (end 171.514398 95.868677) (width 0.381) (layer F.Cu) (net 8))
 (segment (start 172.739398 99.593677) (end 174.009398 99.593677) (width 0.381) (layer F.Cu) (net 9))
 (segment (start 174.009398 101.728677) (end 175.524398 103.243677) (width 0.381) (layer F.Cu) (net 9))
 (segment (start 174.009398 99.593677) (end 174.009398 101.728677) (width 0.381) (layer F.Cu) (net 9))
 (segment (start 181.22 91.613075) (end 179.089398 93.743677) (width 0.381) (layer F.Cu) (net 4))
 (segment (start 179.089398 93.743677) (end 179.089398 94.193677) (width 0.381) (layer F.Cu) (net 4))
 (segment (start 181.22 90.543677) (end 181.22 91.613075) (width 0.381) (layer F.Cu) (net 4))
 (segment (start 181.22 90.543677) (end 181.22 88.003677) (width 0.381) (layer F.Cu) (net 4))
 (segment (start 171.859398 88.003677) (end 171.859398 90.543677) (width 0.381) (layer F.Cu) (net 5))
 (segment (start 177.819398 93.743677) (end 177.819398 94.193677) (width 0.381) (layer F.Cu) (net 5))
 (segment (start 177.8 93.724279) (end 177.819398 93.743677) (width 0.381) (layer F.Cu) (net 5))
 (segment (start 175.895 86.36) (end 176.53 86.995) (width 0.381) (layer F.Cu) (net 5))
 (segment (start 171.84 88.003677) (end 171.84 87.004) (width 0.381) (layer F.Cu) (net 5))
 (segment (start 172.484 86.36) (end 175.895 86.36) (width 0.381) (layer F.Cu) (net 5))
 (segment (start 171.84 87.004) (end 172.484 86.36) (width 0.381) (layer F.Cu) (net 5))
 (segment (start 176.53 86.995) (end 176.53 92.075) (width 0.381) (layer F.Cu) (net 5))
 (segment (start 177.8 93.345) (end 177.8 93.724279) (width 0.381) (layer F.Cu) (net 5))
 (segment (start 176.53 92.075) (end 177.8 93.345) (width 0.381) (layer F.Cu) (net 5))
 (segment (start 179.089398 99.593677) (end 180.359398 99.593677) (width 0.381) (layer F.Cu) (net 12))
 (segment (start 180.359398 99.143677) (end 180.359398 99.593677) (width 0.381) (layer F.Cu) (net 12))
 (segment (start 182.899398 97.918677) (end 181.584398 97.918677) (width 0.381) (layer F.Cu) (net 12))
 (segment (start 181.584398 97.918677) (end 180.359398 99.143677) (width 0.381) (layer F.Cu) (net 12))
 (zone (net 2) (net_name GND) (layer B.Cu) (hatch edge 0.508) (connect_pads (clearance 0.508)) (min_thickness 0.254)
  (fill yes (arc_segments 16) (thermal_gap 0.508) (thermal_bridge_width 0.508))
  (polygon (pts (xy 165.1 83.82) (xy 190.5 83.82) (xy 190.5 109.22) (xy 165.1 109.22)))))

